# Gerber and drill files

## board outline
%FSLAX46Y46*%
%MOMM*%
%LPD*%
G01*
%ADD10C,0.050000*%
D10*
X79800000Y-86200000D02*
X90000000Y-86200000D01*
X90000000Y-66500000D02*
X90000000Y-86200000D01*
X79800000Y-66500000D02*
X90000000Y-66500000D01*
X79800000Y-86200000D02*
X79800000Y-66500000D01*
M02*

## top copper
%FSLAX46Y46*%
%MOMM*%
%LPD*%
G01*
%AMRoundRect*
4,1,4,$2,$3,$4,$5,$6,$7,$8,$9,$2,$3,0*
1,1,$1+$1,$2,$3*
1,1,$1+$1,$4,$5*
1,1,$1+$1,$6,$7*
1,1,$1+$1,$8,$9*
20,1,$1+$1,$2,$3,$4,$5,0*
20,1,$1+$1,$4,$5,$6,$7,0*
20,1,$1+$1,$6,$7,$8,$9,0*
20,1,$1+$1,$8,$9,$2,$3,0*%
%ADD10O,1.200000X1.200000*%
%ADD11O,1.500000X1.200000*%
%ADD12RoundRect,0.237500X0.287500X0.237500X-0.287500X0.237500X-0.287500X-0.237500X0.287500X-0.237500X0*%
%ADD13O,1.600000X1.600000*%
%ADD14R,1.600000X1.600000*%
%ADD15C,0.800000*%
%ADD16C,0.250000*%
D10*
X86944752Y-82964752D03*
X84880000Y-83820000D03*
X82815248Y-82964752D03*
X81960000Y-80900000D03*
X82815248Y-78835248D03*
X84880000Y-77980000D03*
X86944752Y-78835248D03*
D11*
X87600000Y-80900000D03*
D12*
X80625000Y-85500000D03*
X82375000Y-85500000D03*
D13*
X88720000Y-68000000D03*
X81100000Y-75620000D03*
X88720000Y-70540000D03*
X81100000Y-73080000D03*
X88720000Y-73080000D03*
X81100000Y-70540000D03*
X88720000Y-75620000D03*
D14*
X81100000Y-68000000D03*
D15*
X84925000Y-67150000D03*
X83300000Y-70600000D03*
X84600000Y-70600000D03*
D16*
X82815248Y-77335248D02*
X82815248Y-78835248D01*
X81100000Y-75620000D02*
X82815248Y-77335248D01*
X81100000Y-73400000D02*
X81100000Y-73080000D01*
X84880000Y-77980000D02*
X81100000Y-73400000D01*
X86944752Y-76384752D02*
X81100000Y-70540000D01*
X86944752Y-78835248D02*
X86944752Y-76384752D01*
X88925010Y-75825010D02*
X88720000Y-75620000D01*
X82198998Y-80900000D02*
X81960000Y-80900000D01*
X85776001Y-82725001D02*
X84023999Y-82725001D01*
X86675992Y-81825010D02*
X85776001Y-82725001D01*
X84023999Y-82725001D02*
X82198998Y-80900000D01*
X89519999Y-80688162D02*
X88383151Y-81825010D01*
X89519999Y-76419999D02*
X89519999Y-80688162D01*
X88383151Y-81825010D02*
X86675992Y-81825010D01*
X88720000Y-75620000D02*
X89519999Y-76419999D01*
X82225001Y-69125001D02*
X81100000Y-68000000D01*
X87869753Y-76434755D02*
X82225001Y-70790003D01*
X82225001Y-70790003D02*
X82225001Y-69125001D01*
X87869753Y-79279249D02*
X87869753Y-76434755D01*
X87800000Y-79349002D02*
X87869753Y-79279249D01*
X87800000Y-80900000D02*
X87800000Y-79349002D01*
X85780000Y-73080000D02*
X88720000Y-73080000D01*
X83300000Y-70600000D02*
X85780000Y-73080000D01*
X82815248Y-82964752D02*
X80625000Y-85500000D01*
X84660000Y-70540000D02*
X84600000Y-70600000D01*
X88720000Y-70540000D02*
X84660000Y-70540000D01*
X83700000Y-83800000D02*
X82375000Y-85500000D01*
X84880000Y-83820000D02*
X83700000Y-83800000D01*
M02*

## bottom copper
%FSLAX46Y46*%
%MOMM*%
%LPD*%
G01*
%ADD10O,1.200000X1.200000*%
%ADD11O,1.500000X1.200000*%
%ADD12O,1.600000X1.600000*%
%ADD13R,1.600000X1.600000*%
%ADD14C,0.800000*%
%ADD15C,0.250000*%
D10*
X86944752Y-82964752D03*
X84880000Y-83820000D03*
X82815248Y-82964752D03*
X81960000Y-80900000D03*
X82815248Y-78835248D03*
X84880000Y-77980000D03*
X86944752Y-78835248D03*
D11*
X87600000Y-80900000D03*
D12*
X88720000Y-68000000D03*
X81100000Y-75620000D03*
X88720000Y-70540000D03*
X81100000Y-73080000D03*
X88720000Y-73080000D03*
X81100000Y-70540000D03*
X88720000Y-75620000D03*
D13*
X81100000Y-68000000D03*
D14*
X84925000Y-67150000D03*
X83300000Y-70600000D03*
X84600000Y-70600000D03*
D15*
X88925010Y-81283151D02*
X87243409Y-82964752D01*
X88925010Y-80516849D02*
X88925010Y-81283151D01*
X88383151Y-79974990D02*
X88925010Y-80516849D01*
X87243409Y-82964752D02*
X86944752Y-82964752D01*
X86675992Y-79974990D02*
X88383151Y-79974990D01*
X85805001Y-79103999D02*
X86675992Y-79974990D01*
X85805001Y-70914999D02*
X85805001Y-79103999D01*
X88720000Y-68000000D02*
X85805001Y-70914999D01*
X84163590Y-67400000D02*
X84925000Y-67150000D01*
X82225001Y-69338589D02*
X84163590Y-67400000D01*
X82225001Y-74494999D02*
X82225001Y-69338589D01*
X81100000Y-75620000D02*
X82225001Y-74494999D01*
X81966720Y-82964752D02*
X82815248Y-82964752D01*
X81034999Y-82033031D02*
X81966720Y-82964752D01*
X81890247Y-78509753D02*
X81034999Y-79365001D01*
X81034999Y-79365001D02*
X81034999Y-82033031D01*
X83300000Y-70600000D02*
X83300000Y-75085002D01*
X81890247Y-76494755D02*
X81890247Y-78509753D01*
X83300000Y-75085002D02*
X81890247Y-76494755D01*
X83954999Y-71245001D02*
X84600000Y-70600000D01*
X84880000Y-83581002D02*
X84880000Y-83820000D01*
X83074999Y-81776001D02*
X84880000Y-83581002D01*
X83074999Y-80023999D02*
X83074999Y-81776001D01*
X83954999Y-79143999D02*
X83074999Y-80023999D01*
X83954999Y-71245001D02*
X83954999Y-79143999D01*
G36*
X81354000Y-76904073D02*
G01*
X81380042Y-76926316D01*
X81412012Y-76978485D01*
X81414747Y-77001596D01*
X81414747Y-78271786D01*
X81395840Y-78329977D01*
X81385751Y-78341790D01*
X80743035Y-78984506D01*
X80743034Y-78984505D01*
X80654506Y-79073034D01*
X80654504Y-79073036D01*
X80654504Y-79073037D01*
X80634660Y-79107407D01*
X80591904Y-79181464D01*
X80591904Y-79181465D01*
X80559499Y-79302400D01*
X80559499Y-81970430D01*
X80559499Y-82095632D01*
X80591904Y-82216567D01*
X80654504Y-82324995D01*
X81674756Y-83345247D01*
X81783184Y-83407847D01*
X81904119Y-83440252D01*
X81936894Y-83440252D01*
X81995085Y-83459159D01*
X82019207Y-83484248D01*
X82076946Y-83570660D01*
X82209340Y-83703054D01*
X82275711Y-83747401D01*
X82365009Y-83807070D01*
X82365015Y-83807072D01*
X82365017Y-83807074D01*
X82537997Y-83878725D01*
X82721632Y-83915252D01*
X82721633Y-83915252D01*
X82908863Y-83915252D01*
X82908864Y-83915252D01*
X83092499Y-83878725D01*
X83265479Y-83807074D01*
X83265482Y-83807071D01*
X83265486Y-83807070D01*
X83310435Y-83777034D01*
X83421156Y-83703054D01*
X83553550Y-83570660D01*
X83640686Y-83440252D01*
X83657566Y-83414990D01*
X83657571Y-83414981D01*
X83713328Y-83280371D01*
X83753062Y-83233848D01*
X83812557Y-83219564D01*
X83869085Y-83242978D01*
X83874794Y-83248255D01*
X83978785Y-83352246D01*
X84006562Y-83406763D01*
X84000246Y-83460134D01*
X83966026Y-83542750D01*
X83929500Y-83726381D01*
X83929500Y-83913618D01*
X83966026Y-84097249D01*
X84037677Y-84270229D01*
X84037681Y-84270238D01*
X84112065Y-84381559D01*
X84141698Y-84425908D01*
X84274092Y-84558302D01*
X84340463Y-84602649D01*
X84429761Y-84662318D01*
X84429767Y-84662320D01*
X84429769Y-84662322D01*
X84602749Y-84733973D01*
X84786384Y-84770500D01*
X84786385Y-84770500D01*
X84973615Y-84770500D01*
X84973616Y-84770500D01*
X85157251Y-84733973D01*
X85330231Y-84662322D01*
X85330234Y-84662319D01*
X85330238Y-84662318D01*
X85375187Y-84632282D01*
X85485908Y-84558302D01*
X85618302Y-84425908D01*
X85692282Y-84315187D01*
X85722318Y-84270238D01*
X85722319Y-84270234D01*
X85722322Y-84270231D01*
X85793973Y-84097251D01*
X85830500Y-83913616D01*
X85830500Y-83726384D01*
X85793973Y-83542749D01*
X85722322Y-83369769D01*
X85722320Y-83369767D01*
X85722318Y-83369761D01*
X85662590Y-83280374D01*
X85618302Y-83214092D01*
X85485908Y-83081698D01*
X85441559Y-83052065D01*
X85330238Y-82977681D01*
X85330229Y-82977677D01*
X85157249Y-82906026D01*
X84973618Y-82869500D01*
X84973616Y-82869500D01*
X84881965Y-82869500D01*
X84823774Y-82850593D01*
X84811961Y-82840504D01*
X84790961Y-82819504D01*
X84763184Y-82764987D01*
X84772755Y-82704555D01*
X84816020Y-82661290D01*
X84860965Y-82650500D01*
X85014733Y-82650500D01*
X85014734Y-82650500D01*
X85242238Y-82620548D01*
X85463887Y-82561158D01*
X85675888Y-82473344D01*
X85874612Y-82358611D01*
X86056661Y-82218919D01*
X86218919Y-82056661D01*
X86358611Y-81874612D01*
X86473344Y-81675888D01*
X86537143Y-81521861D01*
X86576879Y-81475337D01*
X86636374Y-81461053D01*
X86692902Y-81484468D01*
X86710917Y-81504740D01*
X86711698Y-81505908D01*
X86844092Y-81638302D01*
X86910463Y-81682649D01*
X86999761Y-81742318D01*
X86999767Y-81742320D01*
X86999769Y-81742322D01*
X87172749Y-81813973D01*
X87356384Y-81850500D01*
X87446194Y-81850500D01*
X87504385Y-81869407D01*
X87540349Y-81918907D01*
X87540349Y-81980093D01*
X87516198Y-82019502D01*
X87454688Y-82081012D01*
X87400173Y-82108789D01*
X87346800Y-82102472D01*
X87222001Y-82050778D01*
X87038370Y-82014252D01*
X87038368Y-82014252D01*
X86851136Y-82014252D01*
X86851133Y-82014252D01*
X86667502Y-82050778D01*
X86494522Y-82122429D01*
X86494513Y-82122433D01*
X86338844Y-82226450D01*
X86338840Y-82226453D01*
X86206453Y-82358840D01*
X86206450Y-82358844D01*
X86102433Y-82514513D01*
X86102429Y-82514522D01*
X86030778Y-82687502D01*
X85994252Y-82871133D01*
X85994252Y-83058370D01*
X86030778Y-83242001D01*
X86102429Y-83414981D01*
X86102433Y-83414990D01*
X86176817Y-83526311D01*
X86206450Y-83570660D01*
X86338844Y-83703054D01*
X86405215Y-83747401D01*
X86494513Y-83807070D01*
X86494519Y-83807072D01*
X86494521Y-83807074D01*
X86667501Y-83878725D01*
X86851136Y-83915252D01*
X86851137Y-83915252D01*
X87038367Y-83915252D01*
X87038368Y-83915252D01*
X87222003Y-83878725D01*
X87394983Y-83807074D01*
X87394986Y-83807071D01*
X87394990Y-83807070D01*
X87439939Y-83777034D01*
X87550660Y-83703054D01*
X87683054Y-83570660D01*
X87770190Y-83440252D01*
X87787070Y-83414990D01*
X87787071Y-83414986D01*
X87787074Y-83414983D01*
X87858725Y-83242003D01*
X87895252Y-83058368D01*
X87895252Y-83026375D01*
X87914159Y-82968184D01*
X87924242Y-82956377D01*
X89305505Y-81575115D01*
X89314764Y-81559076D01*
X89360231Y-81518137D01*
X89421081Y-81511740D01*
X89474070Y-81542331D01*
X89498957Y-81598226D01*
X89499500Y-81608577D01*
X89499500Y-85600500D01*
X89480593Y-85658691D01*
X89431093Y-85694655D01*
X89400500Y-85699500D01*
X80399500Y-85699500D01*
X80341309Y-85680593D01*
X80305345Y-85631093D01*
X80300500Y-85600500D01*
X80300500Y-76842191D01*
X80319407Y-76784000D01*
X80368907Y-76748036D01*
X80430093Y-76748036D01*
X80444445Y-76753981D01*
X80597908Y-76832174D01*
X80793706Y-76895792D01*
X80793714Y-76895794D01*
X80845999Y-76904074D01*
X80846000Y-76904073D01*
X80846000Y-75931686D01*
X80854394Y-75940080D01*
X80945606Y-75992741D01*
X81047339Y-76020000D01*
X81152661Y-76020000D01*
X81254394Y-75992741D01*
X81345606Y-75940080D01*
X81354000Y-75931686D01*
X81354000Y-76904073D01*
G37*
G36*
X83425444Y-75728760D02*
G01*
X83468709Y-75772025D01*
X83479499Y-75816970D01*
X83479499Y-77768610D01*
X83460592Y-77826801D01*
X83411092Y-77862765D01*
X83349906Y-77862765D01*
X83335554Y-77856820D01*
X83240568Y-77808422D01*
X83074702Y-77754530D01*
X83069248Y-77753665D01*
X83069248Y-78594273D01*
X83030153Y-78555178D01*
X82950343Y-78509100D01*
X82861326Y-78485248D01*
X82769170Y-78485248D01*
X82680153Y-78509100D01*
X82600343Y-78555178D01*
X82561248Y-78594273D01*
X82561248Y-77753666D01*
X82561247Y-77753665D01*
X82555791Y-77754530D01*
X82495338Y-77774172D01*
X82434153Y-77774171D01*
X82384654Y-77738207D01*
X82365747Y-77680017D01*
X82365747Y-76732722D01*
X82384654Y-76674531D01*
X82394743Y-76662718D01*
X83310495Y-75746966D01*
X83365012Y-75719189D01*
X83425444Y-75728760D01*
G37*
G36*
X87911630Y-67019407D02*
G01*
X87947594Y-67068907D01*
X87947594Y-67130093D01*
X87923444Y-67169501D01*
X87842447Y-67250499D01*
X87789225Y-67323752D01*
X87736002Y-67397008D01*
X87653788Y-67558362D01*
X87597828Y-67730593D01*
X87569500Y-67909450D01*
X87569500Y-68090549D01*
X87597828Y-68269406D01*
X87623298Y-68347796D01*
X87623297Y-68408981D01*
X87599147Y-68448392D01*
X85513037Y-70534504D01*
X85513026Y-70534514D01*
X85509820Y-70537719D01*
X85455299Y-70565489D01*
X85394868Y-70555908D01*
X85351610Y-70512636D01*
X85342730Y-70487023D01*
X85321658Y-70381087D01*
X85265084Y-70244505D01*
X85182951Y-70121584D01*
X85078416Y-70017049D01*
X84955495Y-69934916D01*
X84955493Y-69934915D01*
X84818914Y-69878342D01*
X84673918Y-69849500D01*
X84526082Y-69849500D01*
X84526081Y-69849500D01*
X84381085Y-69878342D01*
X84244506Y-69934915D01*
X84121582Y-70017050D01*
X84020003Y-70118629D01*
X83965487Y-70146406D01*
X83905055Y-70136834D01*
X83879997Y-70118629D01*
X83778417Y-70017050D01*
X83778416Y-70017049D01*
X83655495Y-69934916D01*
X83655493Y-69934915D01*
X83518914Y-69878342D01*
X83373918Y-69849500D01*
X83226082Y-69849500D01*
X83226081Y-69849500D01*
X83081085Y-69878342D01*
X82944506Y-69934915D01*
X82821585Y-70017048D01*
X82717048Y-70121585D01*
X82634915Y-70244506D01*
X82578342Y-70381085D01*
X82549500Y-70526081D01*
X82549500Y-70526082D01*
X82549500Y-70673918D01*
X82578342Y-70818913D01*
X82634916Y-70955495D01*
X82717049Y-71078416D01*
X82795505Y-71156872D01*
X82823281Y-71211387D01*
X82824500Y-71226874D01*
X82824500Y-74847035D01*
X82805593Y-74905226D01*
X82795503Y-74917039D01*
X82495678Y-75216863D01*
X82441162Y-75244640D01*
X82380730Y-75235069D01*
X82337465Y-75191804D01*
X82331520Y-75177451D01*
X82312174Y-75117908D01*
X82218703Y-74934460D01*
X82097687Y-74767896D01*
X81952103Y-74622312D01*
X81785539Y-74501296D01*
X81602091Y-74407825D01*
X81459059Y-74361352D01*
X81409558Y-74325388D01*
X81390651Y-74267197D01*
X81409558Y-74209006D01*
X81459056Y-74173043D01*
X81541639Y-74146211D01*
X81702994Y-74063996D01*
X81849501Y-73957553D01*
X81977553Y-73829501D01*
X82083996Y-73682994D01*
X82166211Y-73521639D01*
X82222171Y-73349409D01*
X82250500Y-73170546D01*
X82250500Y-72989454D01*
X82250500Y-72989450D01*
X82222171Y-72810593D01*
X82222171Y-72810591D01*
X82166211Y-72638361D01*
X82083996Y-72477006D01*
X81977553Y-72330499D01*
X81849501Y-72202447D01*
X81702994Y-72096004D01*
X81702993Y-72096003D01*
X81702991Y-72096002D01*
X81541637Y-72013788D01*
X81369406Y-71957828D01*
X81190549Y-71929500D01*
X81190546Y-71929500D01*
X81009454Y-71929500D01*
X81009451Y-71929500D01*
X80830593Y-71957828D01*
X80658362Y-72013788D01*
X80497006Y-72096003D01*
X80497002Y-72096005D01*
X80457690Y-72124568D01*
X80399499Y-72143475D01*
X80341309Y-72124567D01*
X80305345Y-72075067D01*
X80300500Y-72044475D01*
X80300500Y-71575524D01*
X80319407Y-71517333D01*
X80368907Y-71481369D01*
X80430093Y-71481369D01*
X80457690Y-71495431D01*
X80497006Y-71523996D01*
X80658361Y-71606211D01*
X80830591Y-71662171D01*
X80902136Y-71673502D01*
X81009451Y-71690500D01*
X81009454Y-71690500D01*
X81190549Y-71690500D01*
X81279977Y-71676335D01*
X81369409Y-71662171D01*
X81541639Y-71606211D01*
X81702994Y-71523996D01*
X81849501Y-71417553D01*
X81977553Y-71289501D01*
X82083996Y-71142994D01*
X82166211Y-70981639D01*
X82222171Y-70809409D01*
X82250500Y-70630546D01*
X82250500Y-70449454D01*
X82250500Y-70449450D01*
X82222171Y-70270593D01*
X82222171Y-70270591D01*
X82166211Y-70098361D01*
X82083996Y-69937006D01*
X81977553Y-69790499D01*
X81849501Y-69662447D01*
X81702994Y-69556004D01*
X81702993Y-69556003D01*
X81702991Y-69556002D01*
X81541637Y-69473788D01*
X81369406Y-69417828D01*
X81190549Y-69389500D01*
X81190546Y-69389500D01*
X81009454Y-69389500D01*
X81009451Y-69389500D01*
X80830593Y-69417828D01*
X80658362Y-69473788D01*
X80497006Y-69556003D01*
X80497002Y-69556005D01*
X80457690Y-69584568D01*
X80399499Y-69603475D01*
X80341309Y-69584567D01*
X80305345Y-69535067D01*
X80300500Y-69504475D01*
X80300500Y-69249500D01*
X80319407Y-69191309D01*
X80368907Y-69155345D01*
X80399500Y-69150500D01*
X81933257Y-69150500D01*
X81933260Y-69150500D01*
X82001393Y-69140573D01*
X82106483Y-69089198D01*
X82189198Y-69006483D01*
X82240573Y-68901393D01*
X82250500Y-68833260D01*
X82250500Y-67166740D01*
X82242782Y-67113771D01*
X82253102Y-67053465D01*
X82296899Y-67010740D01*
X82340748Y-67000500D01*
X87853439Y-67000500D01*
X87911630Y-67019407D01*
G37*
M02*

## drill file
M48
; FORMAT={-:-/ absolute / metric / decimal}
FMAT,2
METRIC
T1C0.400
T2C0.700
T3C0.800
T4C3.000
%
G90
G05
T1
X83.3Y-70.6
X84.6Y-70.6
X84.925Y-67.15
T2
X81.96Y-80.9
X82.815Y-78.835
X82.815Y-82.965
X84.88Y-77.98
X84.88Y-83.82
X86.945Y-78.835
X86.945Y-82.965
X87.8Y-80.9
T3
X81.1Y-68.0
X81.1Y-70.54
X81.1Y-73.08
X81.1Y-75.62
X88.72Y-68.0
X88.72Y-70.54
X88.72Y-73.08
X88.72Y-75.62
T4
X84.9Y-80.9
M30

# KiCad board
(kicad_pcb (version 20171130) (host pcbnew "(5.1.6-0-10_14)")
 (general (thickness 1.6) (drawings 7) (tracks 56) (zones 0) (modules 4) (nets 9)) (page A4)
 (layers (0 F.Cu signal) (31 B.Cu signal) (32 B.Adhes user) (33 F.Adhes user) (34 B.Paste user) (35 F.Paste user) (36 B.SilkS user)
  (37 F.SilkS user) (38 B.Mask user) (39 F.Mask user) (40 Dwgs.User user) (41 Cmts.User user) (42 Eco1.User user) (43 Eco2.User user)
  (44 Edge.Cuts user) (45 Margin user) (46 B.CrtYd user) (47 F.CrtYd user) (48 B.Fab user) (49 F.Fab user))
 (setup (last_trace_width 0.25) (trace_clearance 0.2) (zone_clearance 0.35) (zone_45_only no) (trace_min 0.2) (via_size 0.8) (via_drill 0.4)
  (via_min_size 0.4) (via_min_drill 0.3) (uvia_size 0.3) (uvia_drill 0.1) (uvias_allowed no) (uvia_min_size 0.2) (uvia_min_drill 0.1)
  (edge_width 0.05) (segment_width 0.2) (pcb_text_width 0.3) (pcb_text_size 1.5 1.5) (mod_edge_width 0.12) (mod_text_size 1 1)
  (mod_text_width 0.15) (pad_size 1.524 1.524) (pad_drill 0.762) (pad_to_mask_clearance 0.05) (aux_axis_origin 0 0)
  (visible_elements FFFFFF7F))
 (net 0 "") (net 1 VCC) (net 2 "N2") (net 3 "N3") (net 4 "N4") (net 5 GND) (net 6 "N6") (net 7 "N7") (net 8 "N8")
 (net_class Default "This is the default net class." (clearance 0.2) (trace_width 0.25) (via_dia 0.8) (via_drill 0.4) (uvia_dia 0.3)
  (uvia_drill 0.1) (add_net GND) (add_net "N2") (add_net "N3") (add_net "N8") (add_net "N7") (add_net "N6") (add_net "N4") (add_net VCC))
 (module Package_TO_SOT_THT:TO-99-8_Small (layer F.Cu) (at 87.8 80.9 180)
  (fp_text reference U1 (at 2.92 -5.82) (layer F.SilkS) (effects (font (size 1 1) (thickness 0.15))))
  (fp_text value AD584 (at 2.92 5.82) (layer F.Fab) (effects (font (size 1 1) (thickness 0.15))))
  (pad 8 thru_hole oval (at 0.855248 -2.064752 180) (size 1.2 1.2) (drill 0.7) (layers *.Cu *.Mask) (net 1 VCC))
  (pad 7 thru_hole oval (at 2.92 -2.92 180) (size 1.2 1.2) (drill 0.7) (layers *.Cu *.Mask) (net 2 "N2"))
  (pad 6 thru_hole oval (at 4.984752 -2.064752 180) (size 1.2 1.2) (drill 0.7) (layers *.Cu *.Mask) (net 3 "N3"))
  (pad 5 thru_hole oval (at 5.84 0 180) (size 1.2 1.2) (drill 0.7) (layers *.Cu *.Mask) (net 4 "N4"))
  (pad 4 thru_hole oval (at 4.984752 2.064752 180) (size 1.2 1.2) (drill 0.7) (layers *.Cu *.Mask) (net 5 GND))
  (pad 3 thru_hole oval (at 2.92 2.92 180) (size 1.2 1.2) (drill 0.7) (layers *.Cu *.Mask) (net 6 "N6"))
  (pad 2 thru_hole oval (at 0.855248 2.064752 180) (size 1.2 1.2) (drill 0.7) (layers *.Cu *.Mask) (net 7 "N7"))
  (pad 1 thru_hole oval (at 0 0 180) (size 1.5 1.2) (drill 0.7 (offset 0.2 0)) (layers *.Cu *.Mask) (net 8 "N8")))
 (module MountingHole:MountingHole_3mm (layer F.Cu) (at 84.9 80.9)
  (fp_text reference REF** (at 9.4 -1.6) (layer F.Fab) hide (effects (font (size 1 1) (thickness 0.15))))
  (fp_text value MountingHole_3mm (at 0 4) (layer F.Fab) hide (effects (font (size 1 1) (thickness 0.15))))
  (pad 1 np_thru_hole circle (at 0 0) (size 3 3) (drill 3) (layers *.Cu *.Mask)))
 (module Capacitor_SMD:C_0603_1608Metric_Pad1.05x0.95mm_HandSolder (layer F.Cu) (at 81.5 85.5 180)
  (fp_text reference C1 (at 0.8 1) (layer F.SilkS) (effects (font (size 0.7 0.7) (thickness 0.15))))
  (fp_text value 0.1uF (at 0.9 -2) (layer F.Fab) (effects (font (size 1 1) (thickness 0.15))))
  (pad 2 smd roundrect (at 0.875 0 180) (size 1.05 0.95) (layers F.Cu F.Paste F.Mask) (roundrect_rratio 0.25) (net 3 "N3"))
  (pad 1 smd roundrect (at -0.875 0 180) (size 1.05 0.95) (layers F.Cu F.Paste F.Mask) (roundrect_rratio 0.25) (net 2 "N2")))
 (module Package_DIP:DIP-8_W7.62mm (layer F.Cu) (at 81.1 68)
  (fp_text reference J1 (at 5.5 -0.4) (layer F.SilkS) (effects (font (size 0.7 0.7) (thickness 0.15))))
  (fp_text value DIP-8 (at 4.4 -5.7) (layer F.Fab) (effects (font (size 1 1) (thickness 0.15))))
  (pad 8 thru_hole oval (at 7.62 0) (size 1.6 1.6) (drill 0.8) (layers *.Cu *.Mask) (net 1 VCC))
  (pad 4 thru_hole oval (at 0 7.62) (size 1.6 1.6) (drill 0.8) (layers *.Cu *.Mask) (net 5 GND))
  (pad 7 thru_hole oval (at 7.62 2.54) (size 1.6 1.6) (drill 0.8) (layers *.Cu *.Mask) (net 2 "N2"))
  (pad 3 thru_hole oval (at 0 5.08) (size 1.6 1.6) (drill 0.8) (layers *.Cu *.Mask) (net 6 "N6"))
  (pad 6 thru_hole oval (at 7.62 5.08) (size 1.6 1.6) (drill 0.8) (layers *.Cu *.Mask) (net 3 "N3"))
  (pad 2 thru_hole oval (at 0 2.54) (size 1.6 1.6) (drill 0.8) (layers *.Cu *.Mask) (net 7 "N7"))
  (pad 5 thru_hole oval (at 7.62 7.62) (size 1.6 1.6) (drill 0.8) (layers *.Cu *.Mask) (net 4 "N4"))
  (pad 1 thru_hole rect (at 0 0) (size 1.6 1.6) (drill 0.8) (layers *.Cu *.Mask) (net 8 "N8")))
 (gr_line (start 79.8 86.2) (end 90 86.2) (layer Edge.Cuts) (width 0.05))
 (gr_line (start 90 66.5) (end 90 86.2) (layer Edge.Cuts) (width 0.05))
 (gr_line (start 79.8 66.5) (end 90 66.5) (layer Edge.Cuts) (width 0.05))
 (gr_line (start 79.8 86.2) (end 79.8 66.5) (layer Edge.Cuts) (width 0.05))
 (segment (start 88.92501 81.283151) (end 87.243409 82.964752) (width 0.25) (layer B.Cu) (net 1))
 (segment (start 88.92501 80.516849) (end 88.92501 81.283151) (width 0.25) (layer B.Cu) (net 1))
 (segment (start 88.383151 79.97499) (end 88.92501 80.516849) (width 0.25) (layer B.Cu) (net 1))
 (segment (start 87.243409 82.964752) (end 86.944752 82.964752) (width 0.25) (layer B.Cu) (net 1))
 (segment (start 86.675992 79.97499) (end 88.383151 79.97499) (width 0.25) (layer B.Cu) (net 1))
 (segment (start 85.805001 79.103999) (end 86.675992 79.97499) (width 0.25) (layer B.Cu) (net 1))
 (segment (start 85.805001 70.914999) (end 85.805001 79.103999) (width 0.25) (layer B.Cu) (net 1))
 (segment (start 88.72 68) (end 85.805001 70.914999) (width 0.25) (layer B.Cu) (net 1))
 (via (at 84.925 67.15) (size 0.8) (drill 0.4) (layers F.Cu B.Cu) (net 5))
 (segment (start 82.815248 77.335248) (end 82.815248 78.835248) (width 0.25) (layer F.Cu) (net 5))
 (segment (start 81.1 75.62) (end 82.815248 77.335248) (width 0.25) (layer F.Cu) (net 5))
 (segment (start 84.16359 67.4) (end 84.925 67.15) (width 0.25) (layer B.Cu) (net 5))
 (segment (start 82.225001 69.338589) (end 84.16359 67.4) (width 0.25) (layer B.Cu) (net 5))
 (segment (start 82.225001 74.494999) (end 82.225001 69.338589) (width 0.25) (layer B.Cu) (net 5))
 (segment (start 81.1 75.62) (end 82.225001 74.494999) (width 0.25) (layer B.Cu) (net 5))
 (segment (start 81.1 73.4) (end 81.1 73.08) (width 0.25) (layer F.Cu) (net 6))
 (segment (start 84.88 77.98) (end 81.1 73.4) (width 0.25) (layer F.Cu) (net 6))
 (segment (start 86.944752 76.384752) (end 81.1 70.54) (width 0.25) (layer F.Cu) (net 7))
 (segment (start 86.944752 78.835248) (end 86.944752 76.384752) (width 0.25) (layer F.Cu) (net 7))
 (segment (start 88.92501 75.82501) (end 88.72 75.62) (width 0.25) (layer F.Cu) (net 4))
 (segment (start 82.198998 80.9) (end 81.96 80.9) (width 0.25) (layer F.Cu) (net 4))
 (segment (start 85.776001 82.725001) (end 84.023999 82.725001) (width 0.25) (layer F.Cu) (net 4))
 (segment (start 86.675992 81.82501) (end 85.776001 82.725001) (width 0.25) (layer F.Cu) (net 4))
 (segment (start 84.023999 82.725001) (end 82.198998 80.9) (width 0.25) (layer F.Cu) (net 4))
 (segment (start 89.519999 80.688162) (end 88.383151 81.82501) (width 0.25) (layer F.Cu) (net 4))
 (segment (start 89.519999 76.419999) (end 89.519999 80.688162) (width 0.25) (layer F.Cu) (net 4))
 (segment (start 88.383151 81.82501) (end 86.675992 81.82501) (width 0.25) (layer F.Cu) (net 4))
 (segment (start 88.72 75.62) (end 89.519999 76.419999) (width 0.25) (layer F.Cu) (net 4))
 (segment (start 82.225001 69.125001) (end 81.1 68) (width 0.25) (layer F.Cu) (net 8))
 (segment (start 87.869753 76.434755) (end 82.225001 70.790003) (width 0.25) (layer F.Cu) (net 8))
 (segment (start 82.225001 70.790003) (end 82.225001 69.125001) (width 0.25) (layer F.Cu) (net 8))
 (segment (start 87.869753 79.279249) (end 87.869753 76.434755) (width 0.25) (layer F.Cu) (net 8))
 (segment (start 87.8 79.349002) (end 87.869753 79.279249) (width 0.25) (layer F.Cu) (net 8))
 (segment (start 87.8 80.9) (end 87.8 79.349002) (width 0.25) (layer F.Cu) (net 8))
 (via (at 83.3 70.6) (size 0.8) (drill 0.4) (layers F.Cu B.Cu) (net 3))
 (segment (start 85.78 73.08) (end 88.72 73.08) (width 0.25) (layer F.Cu) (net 3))
 (segment (start 83.3 70.6) (end 85.78 73.08) (width 0.25) (layer F.Cu) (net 3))
 (segment (start 82.815248 82.964752) (end 80.625 85.5) (width 0.25) (layer F.Cu) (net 3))
 (segment (start 81.96672 82.964752) (end 82.815248 82.964752) (width 0.25) (layer B.Cu) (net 3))
 (segment (start 81.034999 82.033031) (end 81.96672 82.964752) (width 0.25) (layer B.Cu) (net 3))
 (segment (start 81.890247 78.509753) (end 81.034999 79.365001) (width 0.25) (layer B.Cu) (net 3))
 (segment (start 81.034999 79.365001) (end 81.034999 82.033031) (width 0.25) (layer B.Cu) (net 3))
 (segment (start 83.3 70.6) (end 83.3 75.085002) (width 0.25) (layer B.Cu) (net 3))
 (segment (start 81.890247 76.494755) (end 81.890247 78.509753) (width 0.25) (layer B.Cu) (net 3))
 (segment (start 83.3 75.085002) (end 81.890247 76.494755) (width 0.25) (layer B.Cu) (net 3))
 (via (at 84.6 70.6) (size 0.8) (drill 0.4) (layers F.Cu B.Cu) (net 2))
 (segment (start 84.66 70.54) (end 84.6 70.6) (width 0.25) (layer F.Cu) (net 2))
 (segment (start 88.72 70.54) (end 84.66 70.54) (width 0.25) (layer F.Cu) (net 2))
 (segment (start 83.7 83.8) (end 82.375 85.5) (width 0.25) (layer F.Cu) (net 2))
 (segment (start 84.88 83.82) (end 83.7 83.8) (width 0.25) (layer F.Cu) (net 2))
 (segment (start 83.954999 71.245001) (end 84.6 70.6) (width 0.25) (layer B.Cu) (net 2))
 (segment (start 84.88 83.581002) (end 84.88 83.82) (width 0.25) (layer B.Cu) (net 2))
 (segment (start 83.074999 81.776001) (end 84.88 83.581002) (width 0.25) (layer B.Cu) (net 2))
 (segment (start 83.074999 80.023999) (end 83.074999 81.776001) (width 0.25) (layer B.Cu) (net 2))
 (segment (start 83.954999 79.143999) (end 83.074999 80.023999) (width 0.25) (layer B.Cu) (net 2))
 (segment (start 83.954999 71.245001) (end 83.954999 79.143999) (width 0.25) (layer B.Cu) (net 2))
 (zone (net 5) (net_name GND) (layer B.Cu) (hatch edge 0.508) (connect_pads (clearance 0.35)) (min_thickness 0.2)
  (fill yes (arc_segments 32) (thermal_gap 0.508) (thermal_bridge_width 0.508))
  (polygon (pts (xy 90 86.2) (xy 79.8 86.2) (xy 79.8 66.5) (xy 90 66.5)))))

